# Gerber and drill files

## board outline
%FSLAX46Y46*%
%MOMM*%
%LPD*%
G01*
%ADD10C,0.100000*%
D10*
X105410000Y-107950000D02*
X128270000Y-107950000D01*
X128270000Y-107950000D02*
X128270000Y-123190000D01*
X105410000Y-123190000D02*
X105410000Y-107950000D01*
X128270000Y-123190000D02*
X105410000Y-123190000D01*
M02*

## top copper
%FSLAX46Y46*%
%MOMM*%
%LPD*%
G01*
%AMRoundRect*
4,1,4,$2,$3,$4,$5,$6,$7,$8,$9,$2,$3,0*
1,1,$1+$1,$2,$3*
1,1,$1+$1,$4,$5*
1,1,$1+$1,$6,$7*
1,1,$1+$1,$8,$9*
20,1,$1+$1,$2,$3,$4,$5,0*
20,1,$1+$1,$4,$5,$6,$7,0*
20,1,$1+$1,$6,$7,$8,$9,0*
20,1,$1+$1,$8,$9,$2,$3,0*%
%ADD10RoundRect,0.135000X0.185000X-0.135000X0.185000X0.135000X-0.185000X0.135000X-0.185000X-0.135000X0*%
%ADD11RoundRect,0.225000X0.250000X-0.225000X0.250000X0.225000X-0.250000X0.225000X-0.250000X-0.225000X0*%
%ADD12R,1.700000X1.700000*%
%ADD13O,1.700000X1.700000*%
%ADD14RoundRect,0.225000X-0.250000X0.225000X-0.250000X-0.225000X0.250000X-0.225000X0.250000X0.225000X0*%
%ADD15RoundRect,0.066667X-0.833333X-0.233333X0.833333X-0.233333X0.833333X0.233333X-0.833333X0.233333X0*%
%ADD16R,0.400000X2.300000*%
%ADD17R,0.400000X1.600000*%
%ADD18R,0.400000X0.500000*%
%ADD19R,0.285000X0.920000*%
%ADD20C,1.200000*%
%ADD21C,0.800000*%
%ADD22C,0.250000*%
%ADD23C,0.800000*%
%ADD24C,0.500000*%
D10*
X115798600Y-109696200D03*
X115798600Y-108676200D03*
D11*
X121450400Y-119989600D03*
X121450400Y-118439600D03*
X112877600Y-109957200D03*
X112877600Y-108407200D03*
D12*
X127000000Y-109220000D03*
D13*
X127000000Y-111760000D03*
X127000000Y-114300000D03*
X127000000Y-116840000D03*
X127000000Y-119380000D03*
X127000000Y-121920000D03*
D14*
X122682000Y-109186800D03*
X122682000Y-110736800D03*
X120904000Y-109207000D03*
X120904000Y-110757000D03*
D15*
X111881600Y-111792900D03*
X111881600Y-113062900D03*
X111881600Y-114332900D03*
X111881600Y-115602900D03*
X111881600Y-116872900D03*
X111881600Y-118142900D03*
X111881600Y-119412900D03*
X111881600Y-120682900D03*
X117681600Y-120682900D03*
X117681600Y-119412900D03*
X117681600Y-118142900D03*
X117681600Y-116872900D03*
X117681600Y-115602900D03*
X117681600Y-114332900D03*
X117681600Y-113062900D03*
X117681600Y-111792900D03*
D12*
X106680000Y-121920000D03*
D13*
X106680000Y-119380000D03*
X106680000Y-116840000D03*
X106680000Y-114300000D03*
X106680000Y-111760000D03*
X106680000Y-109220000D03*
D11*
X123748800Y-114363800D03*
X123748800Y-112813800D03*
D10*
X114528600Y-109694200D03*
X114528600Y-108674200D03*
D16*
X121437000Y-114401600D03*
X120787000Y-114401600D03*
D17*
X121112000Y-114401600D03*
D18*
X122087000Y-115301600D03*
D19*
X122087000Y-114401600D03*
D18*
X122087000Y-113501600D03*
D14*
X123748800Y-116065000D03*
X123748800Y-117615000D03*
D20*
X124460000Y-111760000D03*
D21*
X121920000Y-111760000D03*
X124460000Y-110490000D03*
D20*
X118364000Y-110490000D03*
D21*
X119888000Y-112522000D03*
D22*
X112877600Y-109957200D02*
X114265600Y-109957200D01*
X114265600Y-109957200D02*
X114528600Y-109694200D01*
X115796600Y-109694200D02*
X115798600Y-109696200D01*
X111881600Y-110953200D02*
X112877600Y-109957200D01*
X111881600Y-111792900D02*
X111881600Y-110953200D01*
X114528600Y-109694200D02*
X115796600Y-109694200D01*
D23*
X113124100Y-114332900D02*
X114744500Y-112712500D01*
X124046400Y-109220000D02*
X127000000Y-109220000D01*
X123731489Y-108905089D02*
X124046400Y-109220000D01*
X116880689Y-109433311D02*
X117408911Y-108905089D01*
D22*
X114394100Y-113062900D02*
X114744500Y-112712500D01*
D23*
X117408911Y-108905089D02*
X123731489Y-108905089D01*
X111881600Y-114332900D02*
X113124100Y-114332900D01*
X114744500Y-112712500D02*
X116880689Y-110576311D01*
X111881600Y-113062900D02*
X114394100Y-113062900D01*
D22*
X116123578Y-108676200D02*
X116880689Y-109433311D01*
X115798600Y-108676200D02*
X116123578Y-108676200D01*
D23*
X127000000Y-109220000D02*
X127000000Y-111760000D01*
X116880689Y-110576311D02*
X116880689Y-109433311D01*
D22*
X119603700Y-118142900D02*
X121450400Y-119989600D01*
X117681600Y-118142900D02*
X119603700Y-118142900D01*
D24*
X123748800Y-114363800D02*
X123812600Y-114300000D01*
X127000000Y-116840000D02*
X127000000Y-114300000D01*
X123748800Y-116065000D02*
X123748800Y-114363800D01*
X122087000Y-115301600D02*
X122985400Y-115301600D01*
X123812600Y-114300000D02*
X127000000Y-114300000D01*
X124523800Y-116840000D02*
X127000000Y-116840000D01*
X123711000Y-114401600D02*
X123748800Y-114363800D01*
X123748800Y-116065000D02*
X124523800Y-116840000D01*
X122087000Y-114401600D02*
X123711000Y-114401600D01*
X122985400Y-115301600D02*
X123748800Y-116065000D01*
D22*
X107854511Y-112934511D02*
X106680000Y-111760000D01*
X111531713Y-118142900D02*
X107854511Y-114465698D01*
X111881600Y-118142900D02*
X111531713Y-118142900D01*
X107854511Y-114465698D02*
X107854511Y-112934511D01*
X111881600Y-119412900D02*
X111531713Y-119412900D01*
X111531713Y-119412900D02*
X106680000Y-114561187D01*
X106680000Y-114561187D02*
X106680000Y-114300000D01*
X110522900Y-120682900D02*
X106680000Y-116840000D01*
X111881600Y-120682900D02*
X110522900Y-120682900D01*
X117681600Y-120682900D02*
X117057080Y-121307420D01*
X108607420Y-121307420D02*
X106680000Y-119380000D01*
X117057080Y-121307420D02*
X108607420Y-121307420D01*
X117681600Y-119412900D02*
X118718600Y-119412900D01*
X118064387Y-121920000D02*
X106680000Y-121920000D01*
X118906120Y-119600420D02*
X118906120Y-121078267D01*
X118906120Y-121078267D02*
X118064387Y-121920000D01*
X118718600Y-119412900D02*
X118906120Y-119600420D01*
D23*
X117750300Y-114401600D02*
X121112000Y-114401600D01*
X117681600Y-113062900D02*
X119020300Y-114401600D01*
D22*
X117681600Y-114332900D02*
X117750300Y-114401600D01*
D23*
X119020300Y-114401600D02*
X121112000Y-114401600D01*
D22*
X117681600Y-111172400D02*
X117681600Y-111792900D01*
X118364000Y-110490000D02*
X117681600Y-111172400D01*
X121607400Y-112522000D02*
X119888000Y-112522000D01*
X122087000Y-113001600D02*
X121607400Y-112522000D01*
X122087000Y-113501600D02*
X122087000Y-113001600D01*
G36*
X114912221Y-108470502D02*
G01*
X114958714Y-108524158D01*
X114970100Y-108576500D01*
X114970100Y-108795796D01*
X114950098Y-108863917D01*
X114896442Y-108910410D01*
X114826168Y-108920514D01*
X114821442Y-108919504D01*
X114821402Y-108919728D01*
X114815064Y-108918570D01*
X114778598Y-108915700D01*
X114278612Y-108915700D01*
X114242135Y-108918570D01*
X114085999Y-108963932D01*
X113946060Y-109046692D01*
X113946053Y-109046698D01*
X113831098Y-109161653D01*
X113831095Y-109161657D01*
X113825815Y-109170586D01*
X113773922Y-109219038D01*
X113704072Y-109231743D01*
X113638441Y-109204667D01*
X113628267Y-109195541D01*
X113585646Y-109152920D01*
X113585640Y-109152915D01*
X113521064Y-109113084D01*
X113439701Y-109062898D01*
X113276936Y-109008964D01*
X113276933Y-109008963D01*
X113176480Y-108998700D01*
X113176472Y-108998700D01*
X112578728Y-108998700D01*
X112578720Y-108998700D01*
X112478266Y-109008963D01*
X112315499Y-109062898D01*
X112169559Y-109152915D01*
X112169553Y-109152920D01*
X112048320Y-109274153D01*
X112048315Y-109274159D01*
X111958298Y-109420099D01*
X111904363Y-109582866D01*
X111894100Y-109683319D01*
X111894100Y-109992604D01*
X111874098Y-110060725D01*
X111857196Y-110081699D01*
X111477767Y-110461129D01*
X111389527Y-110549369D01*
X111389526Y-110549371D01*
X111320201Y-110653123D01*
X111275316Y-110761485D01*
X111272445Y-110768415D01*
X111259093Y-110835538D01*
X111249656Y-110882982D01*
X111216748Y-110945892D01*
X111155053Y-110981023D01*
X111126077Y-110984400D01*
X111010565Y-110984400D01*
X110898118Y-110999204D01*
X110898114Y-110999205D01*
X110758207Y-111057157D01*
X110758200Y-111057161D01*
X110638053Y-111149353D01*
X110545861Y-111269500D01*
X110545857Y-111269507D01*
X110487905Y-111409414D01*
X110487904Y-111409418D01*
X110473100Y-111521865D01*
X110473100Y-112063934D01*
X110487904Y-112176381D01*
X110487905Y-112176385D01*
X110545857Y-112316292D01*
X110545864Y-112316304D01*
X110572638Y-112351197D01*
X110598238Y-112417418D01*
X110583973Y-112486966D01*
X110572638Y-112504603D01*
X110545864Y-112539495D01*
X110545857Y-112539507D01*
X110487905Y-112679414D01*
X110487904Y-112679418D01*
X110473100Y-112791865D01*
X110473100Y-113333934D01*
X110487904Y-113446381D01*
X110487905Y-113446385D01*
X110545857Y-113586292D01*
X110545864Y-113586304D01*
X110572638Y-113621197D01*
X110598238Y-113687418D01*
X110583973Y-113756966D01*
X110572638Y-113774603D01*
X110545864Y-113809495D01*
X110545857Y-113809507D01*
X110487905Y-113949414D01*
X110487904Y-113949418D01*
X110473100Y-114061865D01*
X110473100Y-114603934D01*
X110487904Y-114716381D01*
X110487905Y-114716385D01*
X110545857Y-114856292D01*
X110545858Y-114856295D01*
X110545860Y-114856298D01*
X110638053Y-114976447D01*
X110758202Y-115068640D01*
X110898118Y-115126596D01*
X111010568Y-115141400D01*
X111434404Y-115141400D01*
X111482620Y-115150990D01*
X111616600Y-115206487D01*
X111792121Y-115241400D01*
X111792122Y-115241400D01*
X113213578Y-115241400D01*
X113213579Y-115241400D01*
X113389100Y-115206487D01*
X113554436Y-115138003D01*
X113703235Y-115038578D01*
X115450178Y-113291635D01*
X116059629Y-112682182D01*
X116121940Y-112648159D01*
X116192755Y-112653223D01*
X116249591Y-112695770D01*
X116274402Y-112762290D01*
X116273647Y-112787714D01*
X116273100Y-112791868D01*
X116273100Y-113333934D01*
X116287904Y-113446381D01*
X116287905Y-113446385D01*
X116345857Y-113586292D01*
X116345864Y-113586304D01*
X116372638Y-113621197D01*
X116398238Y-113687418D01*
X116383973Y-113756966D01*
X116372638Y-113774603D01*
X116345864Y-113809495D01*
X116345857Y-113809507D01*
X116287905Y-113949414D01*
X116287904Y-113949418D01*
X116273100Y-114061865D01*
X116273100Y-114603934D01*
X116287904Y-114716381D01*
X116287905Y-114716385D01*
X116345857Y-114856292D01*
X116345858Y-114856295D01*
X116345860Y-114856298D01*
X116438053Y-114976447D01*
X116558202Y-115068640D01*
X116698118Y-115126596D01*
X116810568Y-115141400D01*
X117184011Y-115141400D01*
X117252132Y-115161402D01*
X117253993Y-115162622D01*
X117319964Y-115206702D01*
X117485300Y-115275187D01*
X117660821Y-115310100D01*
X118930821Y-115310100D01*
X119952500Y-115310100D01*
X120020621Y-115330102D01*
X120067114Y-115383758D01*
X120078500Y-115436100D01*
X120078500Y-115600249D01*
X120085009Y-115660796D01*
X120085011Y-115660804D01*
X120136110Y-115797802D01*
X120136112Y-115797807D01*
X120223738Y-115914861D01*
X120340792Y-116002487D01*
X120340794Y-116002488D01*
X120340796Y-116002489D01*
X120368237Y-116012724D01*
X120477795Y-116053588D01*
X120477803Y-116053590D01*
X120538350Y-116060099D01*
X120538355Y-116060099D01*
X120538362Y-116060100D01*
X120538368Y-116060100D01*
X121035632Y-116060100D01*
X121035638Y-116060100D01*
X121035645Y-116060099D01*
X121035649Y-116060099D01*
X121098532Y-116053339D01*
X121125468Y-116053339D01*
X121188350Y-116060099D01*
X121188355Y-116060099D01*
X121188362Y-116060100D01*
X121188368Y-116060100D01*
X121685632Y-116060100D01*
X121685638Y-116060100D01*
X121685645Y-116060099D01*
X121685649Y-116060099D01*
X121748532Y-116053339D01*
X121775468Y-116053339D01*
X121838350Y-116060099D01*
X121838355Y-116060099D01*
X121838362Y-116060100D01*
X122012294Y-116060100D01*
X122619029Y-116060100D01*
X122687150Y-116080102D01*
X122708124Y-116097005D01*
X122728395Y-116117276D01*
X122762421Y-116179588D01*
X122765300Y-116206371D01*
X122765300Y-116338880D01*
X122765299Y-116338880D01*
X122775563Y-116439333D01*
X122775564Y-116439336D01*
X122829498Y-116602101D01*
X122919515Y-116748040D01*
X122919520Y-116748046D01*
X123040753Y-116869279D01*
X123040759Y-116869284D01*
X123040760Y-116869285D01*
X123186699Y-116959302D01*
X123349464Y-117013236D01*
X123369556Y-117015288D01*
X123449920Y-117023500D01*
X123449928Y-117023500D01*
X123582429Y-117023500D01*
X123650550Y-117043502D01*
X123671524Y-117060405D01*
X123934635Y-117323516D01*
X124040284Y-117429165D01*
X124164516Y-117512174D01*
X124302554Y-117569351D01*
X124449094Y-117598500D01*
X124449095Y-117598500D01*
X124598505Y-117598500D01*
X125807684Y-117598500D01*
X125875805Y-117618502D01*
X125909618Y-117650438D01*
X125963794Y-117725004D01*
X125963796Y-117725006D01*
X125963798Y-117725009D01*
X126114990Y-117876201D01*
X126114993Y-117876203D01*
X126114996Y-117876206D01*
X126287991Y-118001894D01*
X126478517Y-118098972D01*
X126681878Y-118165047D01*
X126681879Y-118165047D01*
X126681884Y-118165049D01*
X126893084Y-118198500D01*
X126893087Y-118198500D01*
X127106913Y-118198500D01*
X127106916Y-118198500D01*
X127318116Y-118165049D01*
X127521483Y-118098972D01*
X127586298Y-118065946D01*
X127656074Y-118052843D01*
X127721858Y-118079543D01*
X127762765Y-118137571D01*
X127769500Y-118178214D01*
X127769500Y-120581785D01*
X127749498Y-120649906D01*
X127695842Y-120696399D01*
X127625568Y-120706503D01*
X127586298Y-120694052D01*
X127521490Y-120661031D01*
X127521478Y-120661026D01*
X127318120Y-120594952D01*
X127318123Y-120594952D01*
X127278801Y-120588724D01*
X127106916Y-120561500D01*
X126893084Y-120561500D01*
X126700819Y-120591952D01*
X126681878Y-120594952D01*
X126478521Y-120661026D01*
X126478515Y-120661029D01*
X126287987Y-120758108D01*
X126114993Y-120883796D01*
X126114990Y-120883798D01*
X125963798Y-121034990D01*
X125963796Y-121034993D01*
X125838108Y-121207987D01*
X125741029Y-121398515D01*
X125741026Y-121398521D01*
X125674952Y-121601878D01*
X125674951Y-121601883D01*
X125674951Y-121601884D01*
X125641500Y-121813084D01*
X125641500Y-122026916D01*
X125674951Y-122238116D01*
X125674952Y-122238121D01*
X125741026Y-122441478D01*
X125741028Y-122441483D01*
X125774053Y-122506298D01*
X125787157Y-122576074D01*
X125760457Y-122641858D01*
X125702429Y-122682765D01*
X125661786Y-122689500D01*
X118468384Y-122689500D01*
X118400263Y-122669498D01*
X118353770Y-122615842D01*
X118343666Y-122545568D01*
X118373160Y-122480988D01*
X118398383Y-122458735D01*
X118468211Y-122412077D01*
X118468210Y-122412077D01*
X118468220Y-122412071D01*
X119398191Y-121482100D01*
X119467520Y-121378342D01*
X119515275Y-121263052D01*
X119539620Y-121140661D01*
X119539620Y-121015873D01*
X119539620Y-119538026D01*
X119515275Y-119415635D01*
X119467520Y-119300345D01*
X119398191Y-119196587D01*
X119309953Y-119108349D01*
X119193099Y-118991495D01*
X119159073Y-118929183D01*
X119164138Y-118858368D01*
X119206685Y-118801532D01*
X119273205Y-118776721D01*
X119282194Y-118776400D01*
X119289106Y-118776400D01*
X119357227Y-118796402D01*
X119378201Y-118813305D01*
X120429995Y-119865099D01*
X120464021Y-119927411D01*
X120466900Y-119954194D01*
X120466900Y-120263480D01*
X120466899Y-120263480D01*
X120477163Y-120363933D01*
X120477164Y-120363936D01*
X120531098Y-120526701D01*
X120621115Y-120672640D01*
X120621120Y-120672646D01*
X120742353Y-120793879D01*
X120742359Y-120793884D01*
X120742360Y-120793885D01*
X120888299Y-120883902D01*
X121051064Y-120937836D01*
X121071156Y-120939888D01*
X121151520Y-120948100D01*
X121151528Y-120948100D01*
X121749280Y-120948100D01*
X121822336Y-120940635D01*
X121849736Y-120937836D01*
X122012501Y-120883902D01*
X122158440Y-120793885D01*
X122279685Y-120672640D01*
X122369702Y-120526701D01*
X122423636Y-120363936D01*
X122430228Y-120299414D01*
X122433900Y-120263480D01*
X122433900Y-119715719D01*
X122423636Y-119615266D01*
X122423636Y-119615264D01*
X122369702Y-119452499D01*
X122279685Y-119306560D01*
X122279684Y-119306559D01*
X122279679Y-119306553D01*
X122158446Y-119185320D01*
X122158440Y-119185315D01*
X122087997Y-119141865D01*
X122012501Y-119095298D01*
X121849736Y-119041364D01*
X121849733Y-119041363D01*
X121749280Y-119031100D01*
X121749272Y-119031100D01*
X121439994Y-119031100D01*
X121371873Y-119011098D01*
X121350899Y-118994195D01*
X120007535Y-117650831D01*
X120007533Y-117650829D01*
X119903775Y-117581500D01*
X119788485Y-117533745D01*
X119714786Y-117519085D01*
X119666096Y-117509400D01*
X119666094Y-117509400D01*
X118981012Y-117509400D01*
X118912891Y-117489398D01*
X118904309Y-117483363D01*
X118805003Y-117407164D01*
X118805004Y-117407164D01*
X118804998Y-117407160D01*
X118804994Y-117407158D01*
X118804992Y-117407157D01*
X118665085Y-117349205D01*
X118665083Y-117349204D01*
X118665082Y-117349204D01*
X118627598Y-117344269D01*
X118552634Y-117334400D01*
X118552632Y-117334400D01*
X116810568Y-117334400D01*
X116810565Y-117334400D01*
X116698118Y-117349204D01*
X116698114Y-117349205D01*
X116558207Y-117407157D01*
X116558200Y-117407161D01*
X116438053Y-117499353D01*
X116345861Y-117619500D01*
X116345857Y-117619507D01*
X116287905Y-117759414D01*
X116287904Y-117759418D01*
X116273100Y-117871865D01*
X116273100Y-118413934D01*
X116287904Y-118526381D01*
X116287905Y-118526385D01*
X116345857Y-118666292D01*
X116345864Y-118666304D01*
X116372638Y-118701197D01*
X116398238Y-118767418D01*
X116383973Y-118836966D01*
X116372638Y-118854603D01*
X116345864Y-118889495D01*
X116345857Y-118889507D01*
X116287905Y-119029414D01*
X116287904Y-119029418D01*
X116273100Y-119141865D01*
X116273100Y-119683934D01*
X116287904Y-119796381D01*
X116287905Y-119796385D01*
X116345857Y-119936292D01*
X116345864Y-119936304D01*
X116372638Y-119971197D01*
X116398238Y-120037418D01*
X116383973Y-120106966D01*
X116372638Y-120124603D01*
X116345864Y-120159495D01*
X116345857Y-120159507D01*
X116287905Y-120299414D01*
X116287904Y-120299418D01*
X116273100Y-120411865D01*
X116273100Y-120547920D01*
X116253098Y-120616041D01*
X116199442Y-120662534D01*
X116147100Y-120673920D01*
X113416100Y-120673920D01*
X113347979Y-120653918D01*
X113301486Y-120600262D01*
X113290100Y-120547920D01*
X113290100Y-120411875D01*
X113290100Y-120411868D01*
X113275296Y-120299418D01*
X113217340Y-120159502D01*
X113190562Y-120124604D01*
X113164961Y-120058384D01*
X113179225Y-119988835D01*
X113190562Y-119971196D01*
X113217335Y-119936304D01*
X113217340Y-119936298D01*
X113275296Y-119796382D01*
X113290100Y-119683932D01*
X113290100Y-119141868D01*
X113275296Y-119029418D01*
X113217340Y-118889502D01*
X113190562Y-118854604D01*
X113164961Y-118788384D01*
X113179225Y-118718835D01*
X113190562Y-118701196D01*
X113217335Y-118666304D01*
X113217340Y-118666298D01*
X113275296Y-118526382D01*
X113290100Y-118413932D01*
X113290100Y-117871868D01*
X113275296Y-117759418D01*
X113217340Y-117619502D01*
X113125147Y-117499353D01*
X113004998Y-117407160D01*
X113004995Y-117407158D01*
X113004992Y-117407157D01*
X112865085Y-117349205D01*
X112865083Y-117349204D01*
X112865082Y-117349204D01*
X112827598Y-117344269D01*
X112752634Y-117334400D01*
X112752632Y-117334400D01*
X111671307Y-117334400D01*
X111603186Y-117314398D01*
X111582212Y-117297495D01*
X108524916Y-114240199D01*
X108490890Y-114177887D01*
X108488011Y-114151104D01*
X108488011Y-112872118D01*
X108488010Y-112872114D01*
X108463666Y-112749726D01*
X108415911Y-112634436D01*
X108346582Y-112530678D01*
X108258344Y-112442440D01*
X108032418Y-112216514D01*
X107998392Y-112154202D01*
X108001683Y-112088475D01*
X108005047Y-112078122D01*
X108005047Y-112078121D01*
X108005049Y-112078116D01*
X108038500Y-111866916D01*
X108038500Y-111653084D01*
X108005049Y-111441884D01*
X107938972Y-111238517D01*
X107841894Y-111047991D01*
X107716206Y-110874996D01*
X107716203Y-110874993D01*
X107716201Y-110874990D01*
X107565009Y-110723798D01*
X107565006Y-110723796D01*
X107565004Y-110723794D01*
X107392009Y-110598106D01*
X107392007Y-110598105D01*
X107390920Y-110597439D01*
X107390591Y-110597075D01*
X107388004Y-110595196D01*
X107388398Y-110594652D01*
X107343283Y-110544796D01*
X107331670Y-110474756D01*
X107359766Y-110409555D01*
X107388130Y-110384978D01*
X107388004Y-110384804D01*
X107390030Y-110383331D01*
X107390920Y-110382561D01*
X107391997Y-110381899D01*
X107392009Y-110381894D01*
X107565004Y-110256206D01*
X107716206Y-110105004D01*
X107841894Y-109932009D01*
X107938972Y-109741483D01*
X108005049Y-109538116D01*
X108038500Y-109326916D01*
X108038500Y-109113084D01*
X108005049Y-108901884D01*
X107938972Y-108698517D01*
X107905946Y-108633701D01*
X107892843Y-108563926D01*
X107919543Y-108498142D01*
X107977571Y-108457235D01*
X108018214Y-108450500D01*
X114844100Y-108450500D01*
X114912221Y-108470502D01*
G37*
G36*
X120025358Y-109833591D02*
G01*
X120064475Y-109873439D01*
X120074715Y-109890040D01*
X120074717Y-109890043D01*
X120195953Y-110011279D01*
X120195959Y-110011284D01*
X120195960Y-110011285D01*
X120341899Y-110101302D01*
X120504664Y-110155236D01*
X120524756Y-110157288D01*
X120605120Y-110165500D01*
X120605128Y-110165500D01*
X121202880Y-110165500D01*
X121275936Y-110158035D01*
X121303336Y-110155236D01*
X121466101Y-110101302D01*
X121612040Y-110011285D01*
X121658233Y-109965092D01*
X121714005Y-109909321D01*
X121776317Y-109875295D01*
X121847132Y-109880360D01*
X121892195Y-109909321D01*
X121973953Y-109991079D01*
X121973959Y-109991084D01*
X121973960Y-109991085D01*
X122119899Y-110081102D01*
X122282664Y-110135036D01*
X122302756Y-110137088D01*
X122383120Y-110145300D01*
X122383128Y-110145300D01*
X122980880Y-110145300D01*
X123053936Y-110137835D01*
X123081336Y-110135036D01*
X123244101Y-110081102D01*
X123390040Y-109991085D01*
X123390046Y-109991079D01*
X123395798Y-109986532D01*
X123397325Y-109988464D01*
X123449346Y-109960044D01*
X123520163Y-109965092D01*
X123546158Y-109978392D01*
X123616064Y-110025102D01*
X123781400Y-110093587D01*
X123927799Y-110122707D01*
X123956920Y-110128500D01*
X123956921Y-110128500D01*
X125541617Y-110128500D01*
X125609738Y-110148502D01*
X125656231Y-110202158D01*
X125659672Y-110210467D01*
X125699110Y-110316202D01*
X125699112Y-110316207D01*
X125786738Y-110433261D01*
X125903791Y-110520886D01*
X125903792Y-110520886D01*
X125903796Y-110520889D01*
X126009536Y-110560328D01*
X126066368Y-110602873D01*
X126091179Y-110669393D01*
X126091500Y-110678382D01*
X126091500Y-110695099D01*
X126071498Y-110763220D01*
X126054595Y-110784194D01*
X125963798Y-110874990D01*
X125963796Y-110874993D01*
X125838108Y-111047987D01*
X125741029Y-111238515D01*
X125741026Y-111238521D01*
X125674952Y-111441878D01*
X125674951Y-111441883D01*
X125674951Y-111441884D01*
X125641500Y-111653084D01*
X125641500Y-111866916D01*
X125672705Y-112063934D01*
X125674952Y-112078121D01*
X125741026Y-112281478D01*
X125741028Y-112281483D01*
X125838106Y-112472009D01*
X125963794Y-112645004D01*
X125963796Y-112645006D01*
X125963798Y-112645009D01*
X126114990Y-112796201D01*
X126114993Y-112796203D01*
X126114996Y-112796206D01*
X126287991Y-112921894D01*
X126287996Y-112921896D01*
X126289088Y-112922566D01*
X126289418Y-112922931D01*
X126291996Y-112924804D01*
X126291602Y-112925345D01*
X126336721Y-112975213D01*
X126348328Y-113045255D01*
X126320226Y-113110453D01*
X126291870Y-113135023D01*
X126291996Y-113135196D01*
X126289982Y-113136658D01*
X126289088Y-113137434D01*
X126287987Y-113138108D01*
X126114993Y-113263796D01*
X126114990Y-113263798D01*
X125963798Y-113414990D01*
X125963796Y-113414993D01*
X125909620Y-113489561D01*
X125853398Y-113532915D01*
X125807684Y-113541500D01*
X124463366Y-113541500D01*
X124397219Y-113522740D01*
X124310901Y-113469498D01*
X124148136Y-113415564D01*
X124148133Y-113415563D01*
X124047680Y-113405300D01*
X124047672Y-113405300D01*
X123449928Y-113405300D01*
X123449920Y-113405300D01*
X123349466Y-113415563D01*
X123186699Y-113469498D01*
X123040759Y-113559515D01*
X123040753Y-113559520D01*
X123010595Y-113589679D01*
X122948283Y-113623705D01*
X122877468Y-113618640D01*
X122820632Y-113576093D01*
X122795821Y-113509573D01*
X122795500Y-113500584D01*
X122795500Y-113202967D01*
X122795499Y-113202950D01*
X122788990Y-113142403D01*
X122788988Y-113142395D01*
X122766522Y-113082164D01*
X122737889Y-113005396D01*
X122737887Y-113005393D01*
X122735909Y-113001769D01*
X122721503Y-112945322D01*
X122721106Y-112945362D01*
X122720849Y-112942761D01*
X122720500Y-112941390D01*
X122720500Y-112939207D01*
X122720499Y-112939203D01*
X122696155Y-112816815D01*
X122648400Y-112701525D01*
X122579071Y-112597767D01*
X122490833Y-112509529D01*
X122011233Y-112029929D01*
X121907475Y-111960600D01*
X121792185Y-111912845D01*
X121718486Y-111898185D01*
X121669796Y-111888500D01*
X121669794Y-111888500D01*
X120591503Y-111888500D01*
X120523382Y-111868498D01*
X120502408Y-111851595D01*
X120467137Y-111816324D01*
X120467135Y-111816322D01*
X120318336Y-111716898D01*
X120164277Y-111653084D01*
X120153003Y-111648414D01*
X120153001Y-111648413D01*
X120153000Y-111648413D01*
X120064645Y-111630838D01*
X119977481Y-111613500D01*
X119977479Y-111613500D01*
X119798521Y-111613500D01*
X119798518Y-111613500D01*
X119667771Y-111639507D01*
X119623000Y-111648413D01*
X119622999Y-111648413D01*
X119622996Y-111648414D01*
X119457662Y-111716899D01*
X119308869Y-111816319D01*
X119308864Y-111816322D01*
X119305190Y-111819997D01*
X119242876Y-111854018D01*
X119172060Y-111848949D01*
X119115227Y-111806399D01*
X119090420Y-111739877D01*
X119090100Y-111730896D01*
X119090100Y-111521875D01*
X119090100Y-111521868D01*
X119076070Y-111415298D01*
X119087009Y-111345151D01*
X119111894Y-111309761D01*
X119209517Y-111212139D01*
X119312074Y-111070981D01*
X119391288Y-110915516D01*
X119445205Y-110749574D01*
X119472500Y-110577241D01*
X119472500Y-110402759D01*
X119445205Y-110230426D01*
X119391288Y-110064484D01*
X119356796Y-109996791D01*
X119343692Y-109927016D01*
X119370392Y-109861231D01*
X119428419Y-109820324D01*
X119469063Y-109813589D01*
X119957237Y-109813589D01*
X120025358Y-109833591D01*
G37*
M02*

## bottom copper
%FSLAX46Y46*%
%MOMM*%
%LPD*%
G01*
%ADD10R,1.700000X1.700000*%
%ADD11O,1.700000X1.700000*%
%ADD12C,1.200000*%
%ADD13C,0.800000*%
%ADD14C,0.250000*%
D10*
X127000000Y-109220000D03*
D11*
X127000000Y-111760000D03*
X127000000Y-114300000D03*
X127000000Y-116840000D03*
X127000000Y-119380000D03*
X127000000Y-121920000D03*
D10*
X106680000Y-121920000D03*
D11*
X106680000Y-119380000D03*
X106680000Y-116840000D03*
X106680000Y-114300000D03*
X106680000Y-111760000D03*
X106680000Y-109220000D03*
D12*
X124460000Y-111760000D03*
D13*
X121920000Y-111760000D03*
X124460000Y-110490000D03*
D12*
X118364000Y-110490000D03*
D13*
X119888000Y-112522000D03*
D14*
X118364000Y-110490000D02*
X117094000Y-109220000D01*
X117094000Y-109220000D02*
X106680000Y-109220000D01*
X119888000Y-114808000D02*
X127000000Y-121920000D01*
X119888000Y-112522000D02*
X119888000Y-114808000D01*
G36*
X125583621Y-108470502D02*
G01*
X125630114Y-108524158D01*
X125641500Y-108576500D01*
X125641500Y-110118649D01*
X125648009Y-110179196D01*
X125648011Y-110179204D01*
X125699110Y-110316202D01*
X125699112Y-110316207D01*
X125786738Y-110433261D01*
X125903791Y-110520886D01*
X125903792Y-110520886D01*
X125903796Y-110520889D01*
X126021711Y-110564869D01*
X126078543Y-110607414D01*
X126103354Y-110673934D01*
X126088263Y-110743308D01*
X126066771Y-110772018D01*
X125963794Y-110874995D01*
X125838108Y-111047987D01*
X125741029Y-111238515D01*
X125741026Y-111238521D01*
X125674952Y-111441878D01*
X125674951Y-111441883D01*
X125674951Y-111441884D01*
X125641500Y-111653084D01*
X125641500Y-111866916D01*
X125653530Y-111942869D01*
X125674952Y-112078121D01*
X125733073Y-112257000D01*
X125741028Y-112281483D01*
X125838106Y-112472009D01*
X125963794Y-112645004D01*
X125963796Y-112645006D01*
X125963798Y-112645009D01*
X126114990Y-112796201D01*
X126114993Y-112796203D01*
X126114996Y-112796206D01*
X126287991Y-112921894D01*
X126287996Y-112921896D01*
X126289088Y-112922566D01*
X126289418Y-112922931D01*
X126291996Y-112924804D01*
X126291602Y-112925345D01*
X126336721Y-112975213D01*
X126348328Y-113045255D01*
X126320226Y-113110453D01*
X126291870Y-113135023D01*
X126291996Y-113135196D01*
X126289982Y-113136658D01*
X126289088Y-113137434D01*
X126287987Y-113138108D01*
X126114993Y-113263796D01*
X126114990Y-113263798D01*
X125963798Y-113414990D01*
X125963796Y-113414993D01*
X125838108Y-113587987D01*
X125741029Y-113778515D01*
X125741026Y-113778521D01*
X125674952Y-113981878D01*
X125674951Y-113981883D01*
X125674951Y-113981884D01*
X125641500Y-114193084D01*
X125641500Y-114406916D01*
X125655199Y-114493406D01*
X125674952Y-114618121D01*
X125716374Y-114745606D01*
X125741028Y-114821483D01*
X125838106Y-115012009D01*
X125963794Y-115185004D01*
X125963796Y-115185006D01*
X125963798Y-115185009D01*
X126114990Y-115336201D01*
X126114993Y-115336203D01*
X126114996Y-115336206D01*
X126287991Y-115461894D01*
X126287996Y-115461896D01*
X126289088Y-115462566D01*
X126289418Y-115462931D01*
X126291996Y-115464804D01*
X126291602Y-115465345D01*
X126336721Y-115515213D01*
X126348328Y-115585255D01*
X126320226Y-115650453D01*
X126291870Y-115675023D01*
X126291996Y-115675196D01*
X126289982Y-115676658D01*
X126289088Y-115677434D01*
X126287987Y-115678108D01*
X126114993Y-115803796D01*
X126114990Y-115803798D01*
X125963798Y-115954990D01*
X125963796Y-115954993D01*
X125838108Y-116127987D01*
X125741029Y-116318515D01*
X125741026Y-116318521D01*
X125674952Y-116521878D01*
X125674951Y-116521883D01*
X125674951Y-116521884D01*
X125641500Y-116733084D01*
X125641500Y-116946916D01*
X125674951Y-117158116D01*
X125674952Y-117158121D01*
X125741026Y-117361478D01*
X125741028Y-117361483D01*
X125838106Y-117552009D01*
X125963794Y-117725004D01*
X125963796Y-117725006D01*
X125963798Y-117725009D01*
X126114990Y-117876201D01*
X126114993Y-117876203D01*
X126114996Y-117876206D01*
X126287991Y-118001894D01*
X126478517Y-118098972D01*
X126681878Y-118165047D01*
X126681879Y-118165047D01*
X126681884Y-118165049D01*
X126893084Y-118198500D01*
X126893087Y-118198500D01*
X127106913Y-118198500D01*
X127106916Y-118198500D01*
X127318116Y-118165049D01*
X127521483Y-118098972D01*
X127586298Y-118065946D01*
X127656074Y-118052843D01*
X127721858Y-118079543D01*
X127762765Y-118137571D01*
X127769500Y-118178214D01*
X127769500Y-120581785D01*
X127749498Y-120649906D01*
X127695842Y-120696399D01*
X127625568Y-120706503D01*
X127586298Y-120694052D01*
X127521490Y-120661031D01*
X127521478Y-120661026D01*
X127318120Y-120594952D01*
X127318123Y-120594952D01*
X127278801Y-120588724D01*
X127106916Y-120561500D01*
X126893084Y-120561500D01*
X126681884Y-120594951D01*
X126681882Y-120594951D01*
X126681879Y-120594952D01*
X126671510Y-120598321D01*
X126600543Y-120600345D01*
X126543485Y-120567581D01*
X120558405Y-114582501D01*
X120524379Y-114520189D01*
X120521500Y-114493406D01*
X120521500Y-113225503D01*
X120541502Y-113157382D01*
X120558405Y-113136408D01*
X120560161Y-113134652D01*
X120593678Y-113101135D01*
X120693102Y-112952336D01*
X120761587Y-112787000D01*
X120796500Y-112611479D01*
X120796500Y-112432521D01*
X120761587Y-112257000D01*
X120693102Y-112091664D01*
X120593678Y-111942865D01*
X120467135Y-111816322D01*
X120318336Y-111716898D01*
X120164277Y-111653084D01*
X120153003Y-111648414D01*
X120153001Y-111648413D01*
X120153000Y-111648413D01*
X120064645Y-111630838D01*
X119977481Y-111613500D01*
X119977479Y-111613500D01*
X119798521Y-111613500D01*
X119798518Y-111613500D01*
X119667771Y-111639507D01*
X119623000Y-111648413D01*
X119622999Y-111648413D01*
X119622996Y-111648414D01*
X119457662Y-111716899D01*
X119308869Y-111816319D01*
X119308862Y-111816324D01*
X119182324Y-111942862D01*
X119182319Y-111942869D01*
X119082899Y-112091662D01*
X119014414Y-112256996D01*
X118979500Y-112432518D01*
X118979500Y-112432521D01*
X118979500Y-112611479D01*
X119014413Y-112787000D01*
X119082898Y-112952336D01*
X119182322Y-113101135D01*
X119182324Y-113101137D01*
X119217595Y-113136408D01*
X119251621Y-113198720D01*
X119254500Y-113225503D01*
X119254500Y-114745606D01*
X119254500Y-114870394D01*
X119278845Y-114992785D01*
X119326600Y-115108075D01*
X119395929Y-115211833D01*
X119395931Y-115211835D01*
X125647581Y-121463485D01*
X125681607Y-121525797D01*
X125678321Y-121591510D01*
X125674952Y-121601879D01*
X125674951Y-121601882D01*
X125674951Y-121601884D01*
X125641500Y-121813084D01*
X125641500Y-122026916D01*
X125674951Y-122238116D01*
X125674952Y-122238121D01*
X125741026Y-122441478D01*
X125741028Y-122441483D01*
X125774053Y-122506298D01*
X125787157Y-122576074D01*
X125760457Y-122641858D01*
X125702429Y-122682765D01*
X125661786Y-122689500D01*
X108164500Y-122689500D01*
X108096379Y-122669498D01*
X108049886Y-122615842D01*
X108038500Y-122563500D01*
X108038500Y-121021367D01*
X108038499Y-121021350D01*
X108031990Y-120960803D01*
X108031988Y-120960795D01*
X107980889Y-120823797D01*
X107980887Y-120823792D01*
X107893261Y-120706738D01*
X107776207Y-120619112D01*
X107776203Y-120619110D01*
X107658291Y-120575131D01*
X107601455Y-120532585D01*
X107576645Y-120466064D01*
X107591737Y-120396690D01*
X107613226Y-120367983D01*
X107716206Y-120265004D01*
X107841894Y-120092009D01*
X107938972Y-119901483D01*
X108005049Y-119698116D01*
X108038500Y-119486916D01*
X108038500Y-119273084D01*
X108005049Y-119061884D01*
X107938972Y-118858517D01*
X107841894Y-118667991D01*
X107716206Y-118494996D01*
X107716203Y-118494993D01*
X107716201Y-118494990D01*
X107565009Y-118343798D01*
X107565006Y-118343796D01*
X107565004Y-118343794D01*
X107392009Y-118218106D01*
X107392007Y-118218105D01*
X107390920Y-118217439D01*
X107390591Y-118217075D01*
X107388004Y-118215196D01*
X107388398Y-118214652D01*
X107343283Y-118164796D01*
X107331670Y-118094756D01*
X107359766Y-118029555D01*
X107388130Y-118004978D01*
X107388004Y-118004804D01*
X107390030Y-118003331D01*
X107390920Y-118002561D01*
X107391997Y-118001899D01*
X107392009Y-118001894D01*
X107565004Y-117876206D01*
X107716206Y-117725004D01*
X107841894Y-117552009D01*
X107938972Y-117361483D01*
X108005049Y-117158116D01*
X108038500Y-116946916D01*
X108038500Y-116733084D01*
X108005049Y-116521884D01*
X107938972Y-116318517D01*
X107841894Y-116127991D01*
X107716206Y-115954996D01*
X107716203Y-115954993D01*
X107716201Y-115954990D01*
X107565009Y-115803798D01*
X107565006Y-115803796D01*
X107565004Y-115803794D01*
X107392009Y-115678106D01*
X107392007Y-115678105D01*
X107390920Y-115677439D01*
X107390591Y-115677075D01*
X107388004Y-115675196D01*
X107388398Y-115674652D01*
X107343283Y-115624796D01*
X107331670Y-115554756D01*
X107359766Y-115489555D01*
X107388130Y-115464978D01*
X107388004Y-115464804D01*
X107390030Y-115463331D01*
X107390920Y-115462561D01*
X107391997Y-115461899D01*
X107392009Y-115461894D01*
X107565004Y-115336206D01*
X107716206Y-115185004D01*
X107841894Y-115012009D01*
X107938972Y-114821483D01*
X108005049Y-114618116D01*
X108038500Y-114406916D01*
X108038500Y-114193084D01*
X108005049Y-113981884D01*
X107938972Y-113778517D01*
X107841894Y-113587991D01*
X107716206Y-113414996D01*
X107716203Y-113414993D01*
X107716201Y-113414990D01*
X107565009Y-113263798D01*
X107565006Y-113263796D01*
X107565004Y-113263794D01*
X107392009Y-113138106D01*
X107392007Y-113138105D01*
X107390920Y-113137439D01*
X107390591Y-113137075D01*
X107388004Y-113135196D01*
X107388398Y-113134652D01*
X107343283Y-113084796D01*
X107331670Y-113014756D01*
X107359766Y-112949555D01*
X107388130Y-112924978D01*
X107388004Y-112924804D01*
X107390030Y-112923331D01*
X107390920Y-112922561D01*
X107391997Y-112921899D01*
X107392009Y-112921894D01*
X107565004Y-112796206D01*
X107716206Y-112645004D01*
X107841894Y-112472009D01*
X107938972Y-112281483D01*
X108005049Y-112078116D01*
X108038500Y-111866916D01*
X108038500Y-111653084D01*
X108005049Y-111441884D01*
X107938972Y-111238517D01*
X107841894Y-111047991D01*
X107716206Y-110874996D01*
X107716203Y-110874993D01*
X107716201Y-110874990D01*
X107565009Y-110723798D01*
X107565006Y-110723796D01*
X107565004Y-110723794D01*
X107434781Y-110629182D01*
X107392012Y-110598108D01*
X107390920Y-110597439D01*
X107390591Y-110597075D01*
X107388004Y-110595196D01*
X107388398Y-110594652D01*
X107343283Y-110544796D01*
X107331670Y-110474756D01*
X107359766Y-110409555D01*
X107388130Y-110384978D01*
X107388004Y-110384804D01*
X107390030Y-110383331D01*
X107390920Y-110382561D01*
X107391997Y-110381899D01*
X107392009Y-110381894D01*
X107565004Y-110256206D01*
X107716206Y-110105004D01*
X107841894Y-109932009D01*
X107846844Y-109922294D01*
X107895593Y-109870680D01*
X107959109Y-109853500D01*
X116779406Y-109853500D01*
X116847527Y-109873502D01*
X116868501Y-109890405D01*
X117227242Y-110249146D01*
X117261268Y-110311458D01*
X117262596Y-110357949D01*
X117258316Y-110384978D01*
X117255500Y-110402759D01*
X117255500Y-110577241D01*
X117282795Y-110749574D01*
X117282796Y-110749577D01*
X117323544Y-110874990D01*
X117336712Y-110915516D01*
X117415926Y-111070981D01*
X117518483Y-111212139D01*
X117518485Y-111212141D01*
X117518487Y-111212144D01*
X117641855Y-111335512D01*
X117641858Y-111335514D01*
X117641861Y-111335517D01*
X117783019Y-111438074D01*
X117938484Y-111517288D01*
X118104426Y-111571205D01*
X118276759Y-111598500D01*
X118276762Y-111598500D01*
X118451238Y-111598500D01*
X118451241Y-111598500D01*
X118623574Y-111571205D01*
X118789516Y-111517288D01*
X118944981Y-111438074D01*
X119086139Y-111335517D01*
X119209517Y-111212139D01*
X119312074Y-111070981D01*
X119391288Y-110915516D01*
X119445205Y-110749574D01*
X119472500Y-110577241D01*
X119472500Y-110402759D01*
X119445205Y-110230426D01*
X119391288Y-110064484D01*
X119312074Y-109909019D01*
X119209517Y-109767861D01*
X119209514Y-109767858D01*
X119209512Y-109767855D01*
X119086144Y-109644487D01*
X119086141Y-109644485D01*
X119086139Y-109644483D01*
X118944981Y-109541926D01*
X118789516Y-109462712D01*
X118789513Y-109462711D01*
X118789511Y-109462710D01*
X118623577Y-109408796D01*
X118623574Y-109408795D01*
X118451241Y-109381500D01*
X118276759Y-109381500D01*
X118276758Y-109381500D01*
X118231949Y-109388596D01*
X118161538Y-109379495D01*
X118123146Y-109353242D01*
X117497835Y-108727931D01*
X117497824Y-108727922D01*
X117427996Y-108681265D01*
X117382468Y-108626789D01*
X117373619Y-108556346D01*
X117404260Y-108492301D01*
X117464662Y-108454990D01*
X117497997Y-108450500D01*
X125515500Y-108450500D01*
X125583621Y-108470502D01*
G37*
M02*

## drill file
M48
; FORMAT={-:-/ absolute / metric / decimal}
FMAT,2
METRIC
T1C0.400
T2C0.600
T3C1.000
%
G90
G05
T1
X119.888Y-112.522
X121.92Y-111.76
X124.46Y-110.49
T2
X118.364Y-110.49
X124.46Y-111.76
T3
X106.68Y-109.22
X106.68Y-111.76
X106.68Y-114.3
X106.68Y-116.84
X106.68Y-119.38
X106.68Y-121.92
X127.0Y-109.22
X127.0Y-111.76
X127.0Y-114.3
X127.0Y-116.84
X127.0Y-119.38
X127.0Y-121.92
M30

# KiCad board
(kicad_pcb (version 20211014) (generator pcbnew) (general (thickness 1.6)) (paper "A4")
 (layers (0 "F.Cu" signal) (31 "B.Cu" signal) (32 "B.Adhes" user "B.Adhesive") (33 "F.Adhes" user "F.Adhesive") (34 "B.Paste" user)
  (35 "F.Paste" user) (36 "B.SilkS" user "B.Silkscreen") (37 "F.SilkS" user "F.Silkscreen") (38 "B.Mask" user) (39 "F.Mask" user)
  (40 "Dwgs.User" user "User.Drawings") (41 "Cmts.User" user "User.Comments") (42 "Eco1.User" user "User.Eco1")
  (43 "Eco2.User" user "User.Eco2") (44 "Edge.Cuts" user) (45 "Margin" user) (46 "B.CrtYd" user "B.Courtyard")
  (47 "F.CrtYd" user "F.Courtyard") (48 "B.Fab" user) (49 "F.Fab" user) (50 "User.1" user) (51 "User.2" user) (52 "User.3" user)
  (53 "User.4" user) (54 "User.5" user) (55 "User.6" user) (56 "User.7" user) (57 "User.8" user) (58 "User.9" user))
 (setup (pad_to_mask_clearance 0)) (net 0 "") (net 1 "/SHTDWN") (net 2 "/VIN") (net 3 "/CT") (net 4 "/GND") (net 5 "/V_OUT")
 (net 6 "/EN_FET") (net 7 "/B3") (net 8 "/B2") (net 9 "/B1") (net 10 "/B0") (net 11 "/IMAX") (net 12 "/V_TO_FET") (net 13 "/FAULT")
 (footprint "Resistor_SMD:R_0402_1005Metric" (layer "F.Cu") (at 115.7986 109.1862 90)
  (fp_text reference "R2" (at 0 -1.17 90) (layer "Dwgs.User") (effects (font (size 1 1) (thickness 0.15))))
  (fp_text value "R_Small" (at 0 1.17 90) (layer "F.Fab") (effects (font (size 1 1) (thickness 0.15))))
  (pad "1" smd roundrect locked (at -0.51 0 90) (size 0.54 0.64) (layers "F.Cu" "F.Paste" "F.Mask") (roundrect_rratio 0.25)
   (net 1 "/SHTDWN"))
  (pad "2" smd roundrect locked (at 0.51 0 90) (size 0.54 0.64) (layers "F.Cu" "F.Paste" "F.Mask") (roundrect_rratio 0.25) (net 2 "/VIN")))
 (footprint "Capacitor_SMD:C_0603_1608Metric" (layer "F.Cu") (at 121.4504 119.2146 90)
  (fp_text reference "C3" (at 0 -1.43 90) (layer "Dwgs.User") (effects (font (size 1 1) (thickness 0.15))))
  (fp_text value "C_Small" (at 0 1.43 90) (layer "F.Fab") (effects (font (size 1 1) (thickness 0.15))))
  (pad "1" smd roundrect locked (at -0.775 0 90) (size 0.9 0.95) (layers "F.Cu" "F.Paste" "F.Mask") (roundrect_rratio 0.25) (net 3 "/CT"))
  (pad "2" smd roundrect locked (at 0.775 0 90) (size 0.9 0.95) (layers "F.Cu" "F.Paste" "F.Mask") (roundrect_rratio 0.25) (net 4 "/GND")))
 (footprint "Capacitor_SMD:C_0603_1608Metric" (layer "F.Cu") (at 112.8776 109.1822 90)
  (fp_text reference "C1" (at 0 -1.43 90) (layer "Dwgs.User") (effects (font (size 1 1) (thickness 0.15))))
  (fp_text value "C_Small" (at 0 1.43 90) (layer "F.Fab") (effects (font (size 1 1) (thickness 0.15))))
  (pad "1" smd roundrect locked (at -0.775 0 90) (size 0.9 0.95) (layers "F.Cu" "F.Paste" "F.Mask") (roundrect_rratio 0.25)
   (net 1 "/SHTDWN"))
  (pad "2" smd roundrect locked (at 0.775 0 90) (size 0.9 0.95) (layers "F.Cu" "F.Paste" "F.Mask") (roundrect_rratio 0.25) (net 4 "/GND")))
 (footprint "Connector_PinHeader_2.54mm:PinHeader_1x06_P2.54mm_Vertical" (layer "F.Cu") (at 127 109.22)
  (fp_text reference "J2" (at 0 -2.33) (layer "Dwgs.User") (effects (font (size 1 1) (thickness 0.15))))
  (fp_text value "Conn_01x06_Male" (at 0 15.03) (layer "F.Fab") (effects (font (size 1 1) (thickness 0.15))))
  (pad "1" thru_hole rect locked (at 0 0) (size 1.7 1.7) (drill 1) (layers *.Cu *.Mask) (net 2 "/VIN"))
  (pad "2" thru_hole oval locked (at 0 2.54) (size 1.7 1.7) (drill 1) (layers *.Cu *.Mask) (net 2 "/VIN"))
  (pad "3" thru_hole oval locked (at 0 5.08) (size 1.7 1.7) (drill 1) (layers *.Cu *.Mask) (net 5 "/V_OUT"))
  (pad "4" thru_hole oval locked (at 0 7.62) (size 1.7 1.7) (drill 1) (layers *.Cu *.Mask) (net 5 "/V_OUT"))
  (pad "5" thru_hole oval locked (at 0 10.16) (size 1.7 1.7) (drill 1) (layers *.Cu *.Mask) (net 4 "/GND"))
  (pad "6" thru_hole oval locked (at 0 12.7) (size 1.7 1.7) (drill 1) (layers *.Cu *.Mask) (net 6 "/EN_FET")))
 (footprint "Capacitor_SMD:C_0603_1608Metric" (layer "F.Cu") (at 122.682 109.9618 -90)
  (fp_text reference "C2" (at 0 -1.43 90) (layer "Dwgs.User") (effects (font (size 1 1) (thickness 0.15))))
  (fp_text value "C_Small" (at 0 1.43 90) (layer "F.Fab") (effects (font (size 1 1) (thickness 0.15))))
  (pad "1" smd roundrect locked (at -0.775 0 270) (size 0.9 0.95) (layers "F.Cu" "F.Paste" "F.Mask") (roundrect_rratio 0.25) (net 2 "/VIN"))
  (pad "2" smd roundrect locked (at 0.775 0 270) (size 0.9 0.95) (layers "F.Cu" "F.Paste" "F.Mask") (roundrect_rratio 0.25) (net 4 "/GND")))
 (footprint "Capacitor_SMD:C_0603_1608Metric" (layer "F.Cu") (at 120.904 109.982 -90)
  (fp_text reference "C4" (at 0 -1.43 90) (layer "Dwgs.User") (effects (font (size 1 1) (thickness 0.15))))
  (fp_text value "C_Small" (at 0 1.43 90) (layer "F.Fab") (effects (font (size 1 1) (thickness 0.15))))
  (pad "1" smd roundrect locked (at -0.775 0 270) (size 0.9 0.95) (layers "F.Cu" "F.Paste" "F.Mask") (roundrect_rratio 0.25) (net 2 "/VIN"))
  (pad "2" smd roundrect locked (at 0.775 0 270) (size 0.9 0.95) (layers "F.Cu" "F.Paste" "F.Mask") (roundrect_rratio 0.25) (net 4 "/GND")))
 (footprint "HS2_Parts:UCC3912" (layer "F.Cu") (at 114.7816 116.2379)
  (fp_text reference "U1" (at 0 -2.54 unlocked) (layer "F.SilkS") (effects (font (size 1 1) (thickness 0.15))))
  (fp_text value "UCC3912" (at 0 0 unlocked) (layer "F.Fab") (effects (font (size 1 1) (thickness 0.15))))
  (pad "1" smd roundrect (at -2.9 -4.445) (size 1.8 0.6) (layers "F.Cu" "F.Paste") (roundrect_rratio 0.1111111111) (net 1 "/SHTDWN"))
  (pad "2" smd roundrect (at -2.9 -3.175) (size 1.8 0.6) (layers "F.Cu" "F.Paste") (roundrect_rratio 0.1111111111) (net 2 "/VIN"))
  (pad "3" smd roundrect (at -2.9 -1.905) (size 1.8 0.6) (layers "F.Cu" "F.Paste") (roundrect_rratio 0.1111111111) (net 2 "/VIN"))
  (pad "4" smd roundrect (at -2.9 -0.635) (size 1.8 0.6) (layers "F.Cu" "F.Paste") (roundrect_rratio 0.1111111111) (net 4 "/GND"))
  (pad "5" smd roundrect (at -2.9 0.635) (size 1.8 0.6) (layers "F.Cu" "F.Paste") (roundrect_rratio 0.1111111111) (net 4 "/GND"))
  (pad "6" smd roundrect (at -2.9 1.905) (size 1.8 0.6) (layers "F.Cu" "F.Paste") (roundrect_rratio 0.1111111111) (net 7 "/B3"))
  (pad "7" smd roundrect (at -2.9 3.175) (size 1.8 0.6) (layers "F.Cu" "F.Paste") (roundrect_rratio 0.1111111111) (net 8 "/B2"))
  (pad "8" smd roundrect (at -2.9 4.445) (size 1.8 0.6) (layers "F.Cu" "F.Paste") (roundrect_rratio 0.1111111111) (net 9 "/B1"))
  (pad "9" smd roundrect (at 2.9 4.445) (size 1.8 0.6) (layers "F.Cu" "F.Paste") (roundrect_rratio 0.1111111111) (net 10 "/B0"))
  (pad "10" smd roundrect (at 2.9 3.175) (size 1.8 0.6) (layers "F.Cu" "F.Paste") (roundrect_rratio 0.1111111111) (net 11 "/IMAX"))
  (pad "11" smd roundrect (at 2.9 1.905) (size 1.8 0.6) (layers "F.Cu" "F.Paste") (roundrect_rratio 0.1111111111) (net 3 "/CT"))
  (pad "12" smd roundrect (at 2.9 0.635) (size 1.8 0.6) (layers "F.Cu" "F.Paste") (roundrect_rratio 0.1111111111) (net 4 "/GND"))
  (pad "13" smd roundrect (at 2.9 -0.635) (size 1.8 0.6) (layers "F.Cu" "F.Paste") (roundrect_rratio 0.1111111111) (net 4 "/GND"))
  (pad "14" smd roundrect (at 2.9 -1.905) (size 1.8 0.6) (layers "F.Cu" "F.Paste") (roundrect_rratio 0.1111111111) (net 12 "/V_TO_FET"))
  (pad "15" smd roundrect (at 2.9 -3.175) (size 1.8 0.6) (layers "F.Cu" "F.Paste") (roundrect_rratio 0.1111111111) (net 12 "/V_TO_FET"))
  (pad "16" smd roundrect (at 2.9 -4.445) (size 1.8 0.6) (layers "F.Cu" "F.Paste") (roundrect_rratio 0.1111111111) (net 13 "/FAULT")))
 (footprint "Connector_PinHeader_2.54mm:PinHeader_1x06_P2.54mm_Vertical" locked (layer "F.Cu") (at 106.68 121.92 180)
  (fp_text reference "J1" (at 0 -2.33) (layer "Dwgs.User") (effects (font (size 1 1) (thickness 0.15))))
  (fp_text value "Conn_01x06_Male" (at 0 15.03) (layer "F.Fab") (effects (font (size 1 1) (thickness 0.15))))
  (pad "1" thru_hole rect locked (at 0 0 180) (size 1.7 1.7) (drill 1) (layers *.Cu *.Mask) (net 11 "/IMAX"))
  (pad "2" thru_hole oval locked (at 0 2.54 180) (size 1.7 1.7) (drill 1) (layers *.Cu *.Mask) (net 10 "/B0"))
  (pad "3" thru_hole oval locked (at 0 5.08 180) (size 1.7 1.7) (drill 1) (layers *.Cu *.Mask) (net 9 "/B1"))
  (pad "4" thru_hole oval locked (at 0 7.62 180) (size 1.7 1.7) (drill 1) (layers *.Cu *.Mask) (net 8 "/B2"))
  (pad "5" thru_hole oval locked (at 0 10.16 180) (size 1.7 1.7) (drill 1) (layers *.Cu *.Mask) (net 7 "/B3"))
  (pad "6" thru_hole oval locked (at 0 12.7 180) (size 1.7 1.7) (drill 1) (layers *.Cu *.Mask) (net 13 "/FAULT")))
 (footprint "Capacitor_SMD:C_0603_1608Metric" (layer "F.Cu") (at 123.7488 113.5888 90)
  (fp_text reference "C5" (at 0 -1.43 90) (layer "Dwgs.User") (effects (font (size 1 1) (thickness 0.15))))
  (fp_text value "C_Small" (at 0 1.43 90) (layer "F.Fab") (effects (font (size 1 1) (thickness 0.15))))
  (pad "1" smd roundrect locked (at -0.775 0 90) (size 0.9 0.95) (layers "F.Cu" "F.Paste" "F.Mask") (roundrect_rratio 0.25) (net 5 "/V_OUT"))
  (pad "2" smd roundrect locked (at 0.775 0 90) (size 0.9 0.95) (layers "F.Cu" "F.Paste" "F.Mask") (roundrect_rratio 0.25) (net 4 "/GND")))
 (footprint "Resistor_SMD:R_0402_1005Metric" (layer "F.Cu") (at 114.5286 109.1842 90)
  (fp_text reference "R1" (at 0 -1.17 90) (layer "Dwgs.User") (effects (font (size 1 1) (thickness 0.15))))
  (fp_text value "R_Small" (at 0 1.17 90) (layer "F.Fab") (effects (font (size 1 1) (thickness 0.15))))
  (pad "1" smd roundrect locked (at -0.51 0 90) (size 0.54 0.64) (layers "F.Cu" "F.Paste" "F.Mask") (roundrect_rratio 0.25)
   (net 1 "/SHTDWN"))
  (pad "2" smd roundrect locked (at 0.51 0 90) (size 0.54 0.64) (layers "F.Cu" "F.Paste" "F.Mask") (roundrect_rratio 0.25) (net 4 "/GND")))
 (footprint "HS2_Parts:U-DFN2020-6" (layer "F.Cu") (at 120.787 114.4016)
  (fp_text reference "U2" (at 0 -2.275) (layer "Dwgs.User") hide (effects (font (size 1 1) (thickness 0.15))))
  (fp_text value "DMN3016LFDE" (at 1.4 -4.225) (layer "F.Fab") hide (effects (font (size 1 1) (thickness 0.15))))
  (pad "1" smd rect locked (at 0.65 0) (size 0.4 2.3) (layers "F.Cu" "F.Paste" "F.Mask") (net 12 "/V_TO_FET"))
  (pad "1" smd rect locked (at 0 0) (size 0.4 2.3) (layers "F.Cu" "F.Paste" "F.Mask") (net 12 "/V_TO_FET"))
  (pad "1" smd rect locked (at 0.325 0) (size 0.4 1.6) (layers "F.Cu" "F.Paste" "F.Mask") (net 12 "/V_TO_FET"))
  (pad "2" smd rect locked (at 1.3 0.9) (size 0.4 0.5) (layers "F.Cu" "F.Paste" "F.Mask") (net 5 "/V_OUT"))
  (pad "2" smd rect locked (at 1.3 0) (size 0.285 0.92) (layers "F.Cu" "F.Paste" "F.Mask") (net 5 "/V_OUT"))
  (pad "3" smd rect locked (at 1.3 -0.9) (size 0.4 0.5) (layers "F.Cu" "F.Paste" "F.Mask") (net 6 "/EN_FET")))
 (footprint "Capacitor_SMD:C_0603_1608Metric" (layer "F.Cu") (at 123.7488 116.84 -90)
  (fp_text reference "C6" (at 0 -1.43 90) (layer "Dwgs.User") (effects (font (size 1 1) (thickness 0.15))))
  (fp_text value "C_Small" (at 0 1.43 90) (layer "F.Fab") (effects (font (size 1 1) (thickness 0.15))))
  (pad "1" smd roundrect locked (at -0.775 0 270) (size 0.9 0.95) (layers "F.Cu" "F.Paste" "F.Mask") (roundrect_rratio 0.25)
   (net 5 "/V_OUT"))
  (pad "2" smd roundrect locked (at 0.775 0 270) (size 0.9 0.95) (layers "F.Cu" "F.Paste" "F.Mask") (roundrect_rratio 0.25) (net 4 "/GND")))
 (gr_line (start 105.41 107.95) (end 128.27 107.95) (layer "Edge.Cuts") (width 0.1))
 (gr_line (start 128.27 107.95) (end 128.27 123.19) (layer "Edge.Cuts") (width 0.1))
 (gr_line (start 105.41 123.19) (end 105.41 107.95) (layer "Edge.Cuts") (width 0.1))
 (gr_line (start 128.27 123.19) (end 105.41 123.19) (layer "Edge.Cuts") (width 0.1))
 (segment (start 112.8776 109.9572) (end 114.2656 109.9572) (width 0.25) (layer "F.Cu") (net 1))
 (segment (start 114.2656 109.9572) (end 114.5286 109.6942) (width 0.25) (layer "F.Cu") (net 1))
 (segment (start 115.7966 109.6942) (end 115.7986 109.6962) (width 0.25) (layer "F.Cu") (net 1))
 (segment (start 111.8816 110.9532) (end 112.8776 109.9572) (width 0.25) (layer "F.Cu") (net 1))
 (segment (start 111.8816 111.7929) (end 111.8816 110.9532) (width 0.25) (layer "F.Cu") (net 1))
 (segment (start 114.5286 109.6942) (end 115.7966 109.6942) (width 0.25) (layer "F.Cu") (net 1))
 (via (at 124.46 111.76) (size 1.2) (drill 0.6) (layers "F.Cu" "B.Cu") (free) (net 4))
 (via (at 121.92 111.76) (size 0.8) (drill 0.4) (layers "F.Cu" "B.Cu") (free) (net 4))
 (via (at 124.46 110.49) (size 0.8) (drill 0.4) (layers "F.Cu" "B.Cu") (free) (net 4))
 (segment (start 113.1241 114.3329) (end 114.7445 112.7125) (width 0.8) (layer "F.Cu") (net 2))
 (segment (start 124.0464 109.22) (end 127 109.22) (width 0.8) (layer "F.Cu") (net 2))
 (segment (start 123.731489 108.905089) (end 124.0464 109.22) (width 0.8) (layer "F.Cu") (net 2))
 (segment (start 116.880689 109.433311) (end 117.408911 108.905089) (width 0.8) (layer "F.Cu") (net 2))
 (segment (start 114.3941 113.0629) (end 114.7445 112.7125) (width 0.25) (layer "F.Cu") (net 2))
 (segment (start 117.408911 108.905089) (end 123.731489 108.905089) (width 0.8) (layer "F.Cu") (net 2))
 (segment (start 111.8816 114.3329) (end 113.1241 114.3329) (width 0.8) (layer "F.Cu") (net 2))
 (segment (start 114.7445 112.7125) (end 116.880689 110.576311) (width 0.8) (layer "F.Cu") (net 2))
 (segment (start 111.8816 113.0629) (end 114.3941 113.0629) (width 0.8) (layer "F.Cu") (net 2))
 (segment (start 116.123578 108.6762) (end 116.880689 109.433311) (width 0.25) (layer "F.Cu") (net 2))
 (segment (start 115.7986 108.6762) (end 116.123578 108.6762) (width 0.25) (layer "F.Cu") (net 2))
 (segment (start 127 109.22) (end 127 111.76) (width 0.8) (layer "F.Cu") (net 2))
 (segment (start 116.880689 110.576311) (end 116.880689 109.433311) (width 0.8) (layer "F.Cu") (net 2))
 (segment (start 119.6037 118.1429) (end 121.4504 119.9896) (width 0.25) (layer "F.Cu") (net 3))
 (segment (start 117.6816 118.1429) (end 119.6037 118.1429) (width 0.25) (layer "F.Cu") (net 3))
 (segment (start 123.7488 114.3638) (end 123.8126 114.3) (width 0.5) (layer "F.Cu") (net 5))
 (segment (start 127 116.84) (end 127 114.3) (width 0.5) (layer "F.Cu") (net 5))
 (segment (start 123.7488 116.065) (end 123.7488 114.3638) (width 0.5) (layer "F.Cu") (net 5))
 (segment (start 122.087 115.3016) (end 122.9854 115.3016) (width 0.5) (layer "F.Cu") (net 5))
 (segment (start 123.8126 114.3) (end 127 114.3) (width 0.5) (layer "F.Cu") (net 5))
 (segment (start 124.5238 116.84) (end 127 116.84) (width 0.5) (layer "F.Cu") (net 5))
 (segment (start 123.711 114.4016) (end 123.7488 114.3638) (width 0.5) (layer "F.Cu") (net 5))
 (segment (start 123.7488 116.065) (end 124.5238 116.84) (width 0.5) (layer "F.Cu") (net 5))
 (segment (start 122.087 114.4016) (end 123.711 114.4016) (width 0.5) (layer "F.Cu") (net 5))
 (segment (start 122.9854 115.3016) (end 123.7488 116.065) (width 0.5) (layer "F.Cu") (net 5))
 (segment (start 107.854511 112.934511) (end 106.68 111.76) (width 0.25) (layer "F.Cu") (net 7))
 (segment (start 111.531713 118.1429) (end 107.854511 114.465698) (width 0.25) (layer "F.Cu") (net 7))
 (segment (start 111.8816 118.1429) (end 111.531713 118.1429) (width 0.25) (layer "F.Cu") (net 7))
 (segment (start 107.854511 114.465698) (end 107.854511 112.934511) (width 0.25) (layer "F.Cu") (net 7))
 (segment (start 111.8816 119.4129) (end 111.531713 119.4129) (width 0.25) (layer "F.Cu") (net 8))
 (segment (start 111.531713 119.4129) (end 106.68 114.561187) (width 0.25) (layer "F.Cu") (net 8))
 (segment (start 106.68 114.561187) (end 106.68 114.3) (width 0.25) (layer "F.Cu") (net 8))
 (segment (start 110.5229 120.6829) (end 106.68 116.84) (width 0.25) (layer "F.Cu") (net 9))
 (segment (start 111.8816 120.6829) (end 110.5229 120.6829) (width 0.25) (layer "F.Cu") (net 9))
 (segment (start 117.6816 120.6829) (end 117.05708 121.30742) (width 0.25) (layer "F.Cu") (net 10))
 (segment (start 108.60742 121.30742) (end 106.68 119.38) (width 0.25) (layer "F.Cu") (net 10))
 (segment (start 117.05708 121.30742) (end 108.60742 121.30742) (width 0.25) (layer "F.Cu") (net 10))
 (segment (start 117.6816 119.4129) (end 118.7186 119.4129) (width 0.25) (layer "F.Cu") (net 11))
 (segment (start 118.064387 121.92) (end 106.68 121.92) (width 0.25) (layer "F.Cu") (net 11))
 (segment (start 118.90612 119.60042) (end 118.90612 121.078267) (width 0.25) (layer "F.Cu") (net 11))
 (segment (start 118.90612 121.078267) (end 118.064387 121.92) (width 0.25) (layer "F.Cu") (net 11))
 (segment (start 118.7186 119.4129) (end 118.90612 119.60042) (width 0.25) (layer "F.Cu") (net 11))
 (segment (start 117.7503 114.4016) (end 121.112 114.4016) (width 0.8) (layer "F.Cu") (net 12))
 (segment (start 117.6816 113.0629) (end 119.0203 114.4016) (width 0.8) (layer "F.Cu") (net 12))
 (segment (start 117.6816 114.3329) (end 117.7503 114.4016) (width 0.25) (layer "F.Cu") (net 12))
 (segment (start 119.0203 114.4016) (end 121.112 114.4016) (width 0.8) (layer "F.Cu") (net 12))
 (segment (start 117.6816 111.1724) (end 117.6816 111.7929) (width 0.25) (layer "F.Cu") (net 13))
 (segment (start 118.364 110.49) (end 117.6816 111.1724) (width 0.25) (layer "F.Cu") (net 13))
 (via (at 118.364 110.49) (size 1.2) (drill 0.6) (layers "F.Cu" "B.Cu") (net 13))
 (segment (start 118.364 110.49) (end 117.094 109.22) (width 0.25) (layer "B.Cu") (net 13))
 (segment (start 117.094 109.22) (end 106.68 109.22) (width 0.25) (layer "B.Cu") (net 13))
 (segment (start 121.6074 112.522) (end 119.888 112.522) (width 0.25) (layer "F.Cu") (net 6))
 (segment (start 122.087 113.0016) (end 121.6074 112.522) (width 0.25) (layer "F.Cu") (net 6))
 (segment (start 122.087 113.5016) (end 122.087 113.0016) (width 0.25) (layer "F.Cu") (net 6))
 (via (at 119.888 112.522) (size 0.8) (drill 0.4) (layers "F.Cu" "B.Cu") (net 6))
 (segment (start 119.888 114.808) (end 127 121.92) (width 0.25) (layer "B.Cu") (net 6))
 (segment (start 119.888 112.522) (end 119.888 114.808) (width 0.25) (layer "B.Cu") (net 6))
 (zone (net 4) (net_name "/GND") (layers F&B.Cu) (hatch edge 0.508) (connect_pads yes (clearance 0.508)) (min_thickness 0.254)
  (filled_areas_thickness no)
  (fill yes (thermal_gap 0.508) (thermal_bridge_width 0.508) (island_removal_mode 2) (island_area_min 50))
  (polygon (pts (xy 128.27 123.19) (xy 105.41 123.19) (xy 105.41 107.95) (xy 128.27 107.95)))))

